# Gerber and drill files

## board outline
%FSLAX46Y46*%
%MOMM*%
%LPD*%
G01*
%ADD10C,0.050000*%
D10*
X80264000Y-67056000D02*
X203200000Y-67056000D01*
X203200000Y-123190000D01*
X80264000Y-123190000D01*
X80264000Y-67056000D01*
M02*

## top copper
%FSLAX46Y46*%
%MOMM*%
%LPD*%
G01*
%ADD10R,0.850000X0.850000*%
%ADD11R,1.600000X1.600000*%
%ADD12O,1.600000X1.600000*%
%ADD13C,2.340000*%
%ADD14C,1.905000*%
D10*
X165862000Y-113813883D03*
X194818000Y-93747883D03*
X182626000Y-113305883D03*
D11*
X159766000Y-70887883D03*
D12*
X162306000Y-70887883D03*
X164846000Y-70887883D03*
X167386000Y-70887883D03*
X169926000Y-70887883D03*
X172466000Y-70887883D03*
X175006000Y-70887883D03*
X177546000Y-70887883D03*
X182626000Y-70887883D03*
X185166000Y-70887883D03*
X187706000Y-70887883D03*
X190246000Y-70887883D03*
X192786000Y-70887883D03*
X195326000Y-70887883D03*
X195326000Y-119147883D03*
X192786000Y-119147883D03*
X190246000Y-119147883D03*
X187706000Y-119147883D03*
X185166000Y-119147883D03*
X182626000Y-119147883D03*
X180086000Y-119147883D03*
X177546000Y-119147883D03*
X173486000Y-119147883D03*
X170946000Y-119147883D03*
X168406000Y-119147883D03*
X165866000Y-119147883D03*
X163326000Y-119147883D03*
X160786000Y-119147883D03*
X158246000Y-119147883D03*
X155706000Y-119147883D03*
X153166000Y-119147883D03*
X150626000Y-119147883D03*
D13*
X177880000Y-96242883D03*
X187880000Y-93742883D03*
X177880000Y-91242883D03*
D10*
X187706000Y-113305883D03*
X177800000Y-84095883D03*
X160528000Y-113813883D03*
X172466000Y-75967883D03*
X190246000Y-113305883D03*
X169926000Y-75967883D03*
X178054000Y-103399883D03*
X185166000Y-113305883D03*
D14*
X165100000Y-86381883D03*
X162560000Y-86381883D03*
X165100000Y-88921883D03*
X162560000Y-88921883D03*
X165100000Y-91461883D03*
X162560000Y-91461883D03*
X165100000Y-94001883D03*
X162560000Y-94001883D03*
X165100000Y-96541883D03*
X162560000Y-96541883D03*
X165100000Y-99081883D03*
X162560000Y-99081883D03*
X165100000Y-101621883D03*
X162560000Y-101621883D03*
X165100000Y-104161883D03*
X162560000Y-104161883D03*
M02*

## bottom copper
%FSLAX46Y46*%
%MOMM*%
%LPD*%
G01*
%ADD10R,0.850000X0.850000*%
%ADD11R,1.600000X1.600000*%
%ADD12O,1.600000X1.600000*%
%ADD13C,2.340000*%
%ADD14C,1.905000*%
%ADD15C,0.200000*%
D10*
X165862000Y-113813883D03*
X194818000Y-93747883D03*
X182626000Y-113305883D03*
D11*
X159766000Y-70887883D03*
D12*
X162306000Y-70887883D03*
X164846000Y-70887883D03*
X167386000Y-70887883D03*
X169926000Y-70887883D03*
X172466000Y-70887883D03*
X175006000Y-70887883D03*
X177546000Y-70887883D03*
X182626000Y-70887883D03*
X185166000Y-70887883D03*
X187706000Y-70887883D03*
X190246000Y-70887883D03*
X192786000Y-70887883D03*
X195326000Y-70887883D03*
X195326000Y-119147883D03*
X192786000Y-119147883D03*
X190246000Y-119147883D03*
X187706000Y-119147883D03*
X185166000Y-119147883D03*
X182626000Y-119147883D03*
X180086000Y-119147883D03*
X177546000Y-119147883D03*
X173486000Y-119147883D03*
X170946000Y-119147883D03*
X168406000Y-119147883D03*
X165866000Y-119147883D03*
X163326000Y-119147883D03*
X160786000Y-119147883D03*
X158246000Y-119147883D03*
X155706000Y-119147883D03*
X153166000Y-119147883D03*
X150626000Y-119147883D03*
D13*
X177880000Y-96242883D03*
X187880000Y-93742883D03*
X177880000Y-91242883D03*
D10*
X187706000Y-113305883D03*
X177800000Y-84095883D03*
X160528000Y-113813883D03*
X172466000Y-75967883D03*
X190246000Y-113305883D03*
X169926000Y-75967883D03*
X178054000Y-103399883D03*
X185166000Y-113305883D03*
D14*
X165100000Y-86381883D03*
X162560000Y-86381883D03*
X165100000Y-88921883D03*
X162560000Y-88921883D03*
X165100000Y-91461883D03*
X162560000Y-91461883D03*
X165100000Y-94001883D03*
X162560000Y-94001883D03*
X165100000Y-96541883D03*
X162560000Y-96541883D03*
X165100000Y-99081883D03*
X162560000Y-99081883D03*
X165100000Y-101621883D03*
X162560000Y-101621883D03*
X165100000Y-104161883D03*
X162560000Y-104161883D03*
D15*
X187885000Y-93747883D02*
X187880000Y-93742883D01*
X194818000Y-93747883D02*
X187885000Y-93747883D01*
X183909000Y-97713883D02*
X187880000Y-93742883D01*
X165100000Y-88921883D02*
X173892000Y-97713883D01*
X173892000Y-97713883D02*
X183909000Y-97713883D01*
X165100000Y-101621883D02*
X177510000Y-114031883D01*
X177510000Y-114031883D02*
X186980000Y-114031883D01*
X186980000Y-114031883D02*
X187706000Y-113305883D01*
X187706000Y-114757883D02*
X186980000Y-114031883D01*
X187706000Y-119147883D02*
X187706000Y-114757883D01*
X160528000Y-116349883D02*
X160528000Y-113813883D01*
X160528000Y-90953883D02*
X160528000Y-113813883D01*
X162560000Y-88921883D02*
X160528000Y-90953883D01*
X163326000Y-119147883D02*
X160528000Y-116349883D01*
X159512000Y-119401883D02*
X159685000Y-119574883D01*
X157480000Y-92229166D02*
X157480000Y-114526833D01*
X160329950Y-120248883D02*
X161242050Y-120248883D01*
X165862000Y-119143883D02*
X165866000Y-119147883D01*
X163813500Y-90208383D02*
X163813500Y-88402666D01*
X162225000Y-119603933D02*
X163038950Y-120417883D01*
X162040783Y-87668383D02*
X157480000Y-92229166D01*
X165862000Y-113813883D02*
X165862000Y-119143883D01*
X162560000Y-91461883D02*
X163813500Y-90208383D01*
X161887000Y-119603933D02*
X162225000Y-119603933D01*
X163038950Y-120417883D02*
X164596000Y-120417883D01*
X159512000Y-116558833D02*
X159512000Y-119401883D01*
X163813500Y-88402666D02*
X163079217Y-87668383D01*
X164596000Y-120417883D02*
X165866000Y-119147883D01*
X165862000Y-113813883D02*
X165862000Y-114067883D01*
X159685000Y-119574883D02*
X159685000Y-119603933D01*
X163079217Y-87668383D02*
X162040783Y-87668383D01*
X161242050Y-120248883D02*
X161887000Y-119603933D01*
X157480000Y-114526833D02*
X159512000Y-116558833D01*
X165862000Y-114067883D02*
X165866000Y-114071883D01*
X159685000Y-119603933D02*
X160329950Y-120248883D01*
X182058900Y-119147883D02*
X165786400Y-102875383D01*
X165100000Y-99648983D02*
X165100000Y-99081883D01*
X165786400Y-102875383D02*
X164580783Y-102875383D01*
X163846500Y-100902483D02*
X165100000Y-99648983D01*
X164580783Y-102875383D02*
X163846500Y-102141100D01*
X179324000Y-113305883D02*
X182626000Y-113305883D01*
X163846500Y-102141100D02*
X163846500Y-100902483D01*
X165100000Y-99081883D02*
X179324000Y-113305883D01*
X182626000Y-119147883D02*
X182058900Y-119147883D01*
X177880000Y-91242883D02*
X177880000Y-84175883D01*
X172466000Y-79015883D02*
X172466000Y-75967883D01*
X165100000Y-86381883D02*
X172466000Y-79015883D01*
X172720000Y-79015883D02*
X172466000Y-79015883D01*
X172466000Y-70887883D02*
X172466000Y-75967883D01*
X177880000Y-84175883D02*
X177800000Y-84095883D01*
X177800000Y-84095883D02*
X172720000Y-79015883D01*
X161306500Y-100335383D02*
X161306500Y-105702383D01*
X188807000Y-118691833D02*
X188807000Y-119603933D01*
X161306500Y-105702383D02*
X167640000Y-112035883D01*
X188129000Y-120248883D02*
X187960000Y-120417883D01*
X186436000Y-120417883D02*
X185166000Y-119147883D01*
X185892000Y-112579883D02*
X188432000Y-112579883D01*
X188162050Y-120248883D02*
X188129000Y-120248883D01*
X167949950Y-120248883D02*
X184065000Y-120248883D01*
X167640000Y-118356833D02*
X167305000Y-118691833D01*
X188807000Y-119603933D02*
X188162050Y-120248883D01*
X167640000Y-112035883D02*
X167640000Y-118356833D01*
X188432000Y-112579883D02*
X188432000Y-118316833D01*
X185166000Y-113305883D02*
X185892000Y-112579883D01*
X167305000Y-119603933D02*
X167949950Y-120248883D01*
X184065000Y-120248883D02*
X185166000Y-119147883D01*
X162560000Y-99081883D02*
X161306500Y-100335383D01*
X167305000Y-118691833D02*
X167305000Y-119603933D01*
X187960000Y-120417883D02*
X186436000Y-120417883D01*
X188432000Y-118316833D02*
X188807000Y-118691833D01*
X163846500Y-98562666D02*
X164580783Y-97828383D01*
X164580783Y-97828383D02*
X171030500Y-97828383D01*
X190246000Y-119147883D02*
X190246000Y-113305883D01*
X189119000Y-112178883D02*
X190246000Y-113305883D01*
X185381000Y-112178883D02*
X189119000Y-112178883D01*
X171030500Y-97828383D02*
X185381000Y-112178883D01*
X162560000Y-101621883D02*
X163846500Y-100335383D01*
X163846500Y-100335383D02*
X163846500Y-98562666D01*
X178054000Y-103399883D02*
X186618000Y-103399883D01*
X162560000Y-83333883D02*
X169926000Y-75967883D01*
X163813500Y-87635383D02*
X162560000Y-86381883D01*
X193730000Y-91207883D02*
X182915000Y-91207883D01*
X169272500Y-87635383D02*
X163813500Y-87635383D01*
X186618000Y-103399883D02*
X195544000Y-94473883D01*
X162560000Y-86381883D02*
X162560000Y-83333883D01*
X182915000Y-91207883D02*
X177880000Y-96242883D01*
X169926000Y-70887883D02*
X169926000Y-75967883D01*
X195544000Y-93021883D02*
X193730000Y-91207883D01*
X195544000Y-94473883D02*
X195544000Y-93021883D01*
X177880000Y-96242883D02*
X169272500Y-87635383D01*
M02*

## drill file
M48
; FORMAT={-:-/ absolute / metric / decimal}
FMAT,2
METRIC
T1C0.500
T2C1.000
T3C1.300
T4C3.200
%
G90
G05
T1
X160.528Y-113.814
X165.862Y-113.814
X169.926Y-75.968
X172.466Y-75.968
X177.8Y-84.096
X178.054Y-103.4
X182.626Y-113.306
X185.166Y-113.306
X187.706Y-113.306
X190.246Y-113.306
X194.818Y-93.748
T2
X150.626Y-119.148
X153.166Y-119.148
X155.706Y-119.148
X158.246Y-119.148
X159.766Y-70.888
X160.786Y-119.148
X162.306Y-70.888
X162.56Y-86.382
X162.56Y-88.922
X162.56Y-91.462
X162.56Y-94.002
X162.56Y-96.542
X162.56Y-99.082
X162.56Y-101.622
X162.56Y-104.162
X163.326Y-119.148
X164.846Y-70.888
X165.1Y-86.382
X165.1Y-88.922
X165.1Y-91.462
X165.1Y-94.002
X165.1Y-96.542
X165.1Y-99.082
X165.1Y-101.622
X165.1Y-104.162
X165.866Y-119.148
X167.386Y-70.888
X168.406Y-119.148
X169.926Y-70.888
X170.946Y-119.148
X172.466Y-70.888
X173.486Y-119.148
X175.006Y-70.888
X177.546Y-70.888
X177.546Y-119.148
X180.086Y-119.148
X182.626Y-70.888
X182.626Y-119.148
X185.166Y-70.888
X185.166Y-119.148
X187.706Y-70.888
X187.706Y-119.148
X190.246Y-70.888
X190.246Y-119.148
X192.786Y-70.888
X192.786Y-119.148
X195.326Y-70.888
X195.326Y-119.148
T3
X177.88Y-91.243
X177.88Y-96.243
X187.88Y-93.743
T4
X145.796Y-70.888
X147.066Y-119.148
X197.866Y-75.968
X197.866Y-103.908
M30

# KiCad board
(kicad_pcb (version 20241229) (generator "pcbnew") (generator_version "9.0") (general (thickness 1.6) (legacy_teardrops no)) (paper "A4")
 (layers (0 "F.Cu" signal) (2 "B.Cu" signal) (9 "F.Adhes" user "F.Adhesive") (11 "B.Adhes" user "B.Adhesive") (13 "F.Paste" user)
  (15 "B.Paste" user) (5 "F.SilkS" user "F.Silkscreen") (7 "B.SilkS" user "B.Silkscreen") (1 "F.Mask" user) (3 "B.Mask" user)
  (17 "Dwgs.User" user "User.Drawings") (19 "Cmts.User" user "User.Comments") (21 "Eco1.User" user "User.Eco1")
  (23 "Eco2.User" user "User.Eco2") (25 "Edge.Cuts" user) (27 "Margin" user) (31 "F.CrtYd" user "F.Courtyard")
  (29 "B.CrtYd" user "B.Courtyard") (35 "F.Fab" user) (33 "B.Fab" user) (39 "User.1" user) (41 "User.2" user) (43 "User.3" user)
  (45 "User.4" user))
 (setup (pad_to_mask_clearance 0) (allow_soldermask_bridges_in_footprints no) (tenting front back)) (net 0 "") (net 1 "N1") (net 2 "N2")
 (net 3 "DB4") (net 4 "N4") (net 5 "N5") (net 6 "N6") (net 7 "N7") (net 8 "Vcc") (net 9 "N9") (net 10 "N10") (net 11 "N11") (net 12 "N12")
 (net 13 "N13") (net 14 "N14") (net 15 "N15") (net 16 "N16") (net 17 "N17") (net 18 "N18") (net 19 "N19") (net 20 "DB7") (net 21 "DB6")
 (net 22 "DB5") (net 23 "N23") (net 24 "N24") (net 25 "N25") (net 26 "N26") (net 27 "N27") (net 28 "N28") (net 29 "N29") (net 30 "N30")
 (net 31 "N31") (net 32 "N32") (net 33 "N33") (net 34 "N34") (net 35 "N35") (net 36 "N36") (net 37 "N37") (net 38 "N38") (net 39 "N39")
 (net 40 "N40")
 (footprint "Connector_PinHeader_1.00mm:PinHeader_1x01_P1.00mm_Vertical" (layer "F.Cu") (at 165.862 113.813883)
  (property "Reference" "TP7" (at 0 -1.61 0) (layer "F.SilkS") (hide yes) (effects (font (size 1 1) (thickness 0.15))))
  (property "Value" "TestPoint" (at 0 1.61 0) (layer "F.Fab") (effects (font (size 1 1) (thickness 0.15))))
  (pad "1" thru_hole rect (at 0 0) (size 0.85 0.85) (drill 0.5) (layers "*.Cu" "*.Mask") (remove_unused_layers no) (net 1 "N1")))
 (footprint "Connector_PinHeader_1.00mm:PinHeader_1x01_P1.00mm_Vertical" (layer "F.Cu") (at 194.818 93.747883)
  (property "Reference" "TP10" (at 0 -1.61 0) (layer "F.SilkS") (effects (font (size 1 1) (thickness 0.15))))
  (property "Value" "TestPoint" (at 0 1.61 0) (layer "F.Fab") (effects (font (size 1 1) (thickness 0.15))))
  (pad "1" thru_hole rect (at 0 0) (size 0.85 0.85) (drill 0.5) (layers "*.Cu" "*.Mask") (remove_unused_layers no) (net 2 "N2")))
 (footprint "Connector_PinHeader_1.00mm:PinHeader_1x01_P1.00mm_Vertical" (layer "F.Cu") (at 182.626 113.305883)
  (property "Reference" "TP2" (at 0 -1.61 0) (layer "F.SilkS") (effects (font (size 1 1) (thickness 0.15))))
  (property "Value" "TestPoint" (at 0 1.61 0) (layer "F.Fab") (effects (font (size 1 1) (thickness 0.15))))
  (pad "1" thru_hole rect (at 0 0) (size 0.85 0.85) (drill 0.5) (layers "*.Cu" "*.Mask") (remove_unused_layers no) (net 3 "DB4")))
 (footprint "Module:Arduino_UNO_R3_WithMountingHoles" (layer "F.Cu") (at 159.766 70.887883)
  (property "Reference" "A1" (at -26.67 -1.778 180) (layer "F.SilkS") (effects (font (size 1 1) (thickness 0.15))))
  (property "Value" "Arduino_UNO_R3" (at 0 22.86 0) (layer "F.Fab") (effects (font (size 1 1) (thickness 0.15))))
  (pad "" np_thru_hole circle (at -13.97 0 90) (size 3.2 3.2) (drill 3.2) (layers "*.Cu" "*.Mask"))
  (pad "" np_thru_hole circle (at -12.7 48.26 90) (size 3.2 3.2) (drill 3.2) (layers "*.Cu" "*.Mask"))
  (pad "" np_thru_hole circle (at 38.1 5.08 90) (size 3.2 3.2) (drill 3.2) (layers "*.Cu" "*.Mask"))
  (pad "" np_thru_hole circle (at 38.1 33.02 90) (size 3.2 3.2) (drill 3.2) (layers "*.Cu" "*.Mask"))
  (pad "1" thru_hole rect (at 0 0 90) (size 1.6 1.6) (drill 1) (layers "*.Cu" "*.Mask") (remove_unused_layers no) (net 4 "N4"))
  (pad "2" thru_hole oval (at 2.54 0 90) (size 1.6 1.6) (drill 1) (layers "*.Cu" "*.Mask") (remove_unused_layers no) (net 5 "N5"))
  (pad "3" thru_hole oval (at 5.08 0 90) (size 1.6 1.6) (drill 1) (layers "*.Cu" "*.Mask") (remove_unused_layers no) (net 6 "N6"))
  (pad "4" thru_hole oval (at 7.62 0 90) (size 1.6 1.6) (drill 1) (layers "*.Cu" "*.Mask") (remove_unused_layers no) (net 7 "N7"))
  (pad "5" thru_hole oval (at 10.16 0 90) (size 1.6 1.6) (drill 1) (layers "*.Cu" "*.Mask") (remove_unused_layers no) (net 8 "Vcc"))
  (pad "6" thru_hole oval (at 12.7 0 90) (size 1.6 1.6) (drill 1) (layers "*.Cu" "*.Mask") (remove_unused_layers no) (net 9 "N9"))
  (pad "7" thru_hole oval (at 15.24 0 90) (size 1.6 1.6) (drill 1) (layers "*.Cu" "*.Mask") (remove_unused_layers no) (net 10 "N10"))
  (pad "8" thru_hole oval (at 17.78 0 90) (size 1.6 1.6) (drill 1) (layers "*.Cu" "*.Mask") (remove_unused_layers no) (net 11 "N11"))
  (pad "9" thru_hole oval (at 22.86 0 90) (size 1.6 1.6) (drill 1) (layers "*.Cu" "*.Mask") (remove_unused_layers no) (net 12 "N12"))
  (pad "10" thru_hole oval (at 25.4 0 90) (size 1.6 1.6) (drill 1) (layers "*.Cu" "*.Mask") (remove_unused_layers no) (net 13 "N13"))
  (pad "11" thru_hole oval (at 27.94 0 90) (size 1.6 1.6) (drill 1) (layers "*.Cu" "*.Mask") (remove_unused_layers no) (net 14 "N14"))
  (pad "12" thru_hole oval (at 30.48 0 90) (size 1.6 1.6) (drill 1) (layers "*.Cu" "*.Mask") (remove_unused_layers no) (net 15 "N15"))
  (pad "13" thru_hole oval (at 33.02 0 90) (size 1.6 1.6) (drill 1) (layers "*.Cu" "*.Mask") (remove_unused_layers no) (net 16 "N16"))
  (pad "14" thru_hole oval (at 35.56 0 90) (size 1.6 1.6) (drill 1) (layers "*.Cu" "*.Mask") (remove_unused_layers no) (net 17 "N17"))
  (pad "15" thru_hole oval (at 35.56 48.26 90) (size 1.6 1.6) (drill 1) (layers "*.Cu" "*.Mask") (remove_unused_layers no) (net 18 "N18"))
  (pad "16" thru_hole oval (at 33.02 48.26 90) (size 1.6 1.6) (drill 1) (layers "*.Cu" "*.Mask") (remove_unused_layers no) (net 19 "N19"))
  (pad "17" thru_hole oval (at 30.48 48.26 90) (size 1.6 1.6) (drill 1) (layers "*.Cu" "*.Mask") (remove_unused_layers no) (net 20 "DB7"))
  (pad "18" thru_hole oval (at 27.94 48.26 90) (size 1.6 1.6) (drill 1) (layers "*.Cu" "*.Mask") (remove_unused_layers no) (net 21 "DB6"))
  (pad "19" thru_hole oval (at 25.4 48.26 90) (size 1.6 1.6) (drill 1) (layers "*.Cu" "*.Mask") (remove_unused_layers no) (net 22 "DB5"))
  (pad "20" thru_hole oval (at 22.86 48.26 90) (size 1.6 1.6) (drill 1) (layers "*.Cu" "*.Mask") (remove_unused_layers no) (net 3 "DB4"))
  (pad "21" thru_hole oval (at 20.32 48.26 90) (size 1.6 1.6) (drill 1) (layers "*.Cu" "*.Mask") (remove_unused_layers no) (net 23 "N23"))
  (pad "22" thru_hole oval (at 17.78 48.26 90) (size 1.6 1.6) (drill 1) (layers "*.Cu" "*.Mask") (remove_unused_layers no) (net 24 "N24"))
  (pad "23" thru_hole oval (at 13.72 48.26 90) (size 1.6 1.6) (drill 1) (layers "*.Cu" "*.Mask") (remove_unused_layers no) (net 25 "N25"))
  (pad "24" thru_hole oval (at 11.18 48.26 90) (size 1.6 1.6) (drill 1) (layers "*.Cu" "*.Mask") (remove_unused_layers no) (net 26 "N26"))
  (pad "25" thru_hole oval (at 8.64 48.26 90) (size 1.6 1.6) (drill 1) (layers "*.Cu" "*.Mask") (remove_unused_layers no) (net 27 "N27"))
  (pad "26" thru_hole oval (at 6.1 48.26 90) (size 1.6 1.6) (drill 1) (layers "*.Cu" "*.Mask") (remove_unused_layers no) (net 1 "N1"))
  (pad "27" thru_hole oval (at 3.56 48.26 90) (size 1.6 1.6) (drill 1) (layers "*.Cu" "*.Mask") (remove_unused_layers no) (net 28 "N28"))
  (pad "28" thru_hole oval (at 1.02 48.26 90) (size 1.6 1.6) (drill 1) (layers "*.Cu" "*.Mask") (remove_unused_layers no) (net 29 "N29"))
  (pad "29" thru_hole oval (at -1.52 48.26 90) (size 1.6 1.6) (drill 1) (layers "*.Cu" "*.Mask") (remove_unused_layers no) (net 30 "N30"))
  (pad "30" thru_hole oval (at -4.06 48.26 90) (size 1.6 1.6) (drill 1) (layers "*.Cu" "*.Mask") (remove_unused_layers no) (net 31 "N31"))
  (pad "31" thru_hole oval (at -6.6 48.26 90) (size 1.6 1.6) (drill 1) (layers "*.Cu" "*.Mask") (remove_unused_layers no) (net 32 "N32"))
  (pad "32" thru_hole oval (at -9.14 48.26 90) (size 1.6 1.6) (drill 1) (layers "*.Cu" "*.Mask") (remove_unused_layers no) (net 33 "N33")))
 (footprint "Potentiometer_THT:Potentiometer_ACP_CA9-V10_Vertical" (layer "F.Cu") (at 177.88 96.242883)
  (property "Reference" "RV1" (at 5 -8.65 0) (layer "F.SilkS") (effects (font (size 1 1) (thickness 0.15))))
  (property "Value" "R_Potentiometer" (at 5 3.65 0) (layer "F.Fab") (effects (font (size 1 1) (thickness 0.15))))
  (pad "1" thru_hole circle (at 0 0) (size 2.34 2.34) (drill 1.3) (layers "*.Cu" "*.Mask") (remove_unused_layers no) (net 8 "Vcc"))
  (pad "2" thru_hole circle (at 10 -2.5) (size 2.34 2.34) (drill 1.3) (layers "*.Cu" "*.Mask") (remove_unused_layers no) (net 2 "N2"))
  (pad "3" thru_hole circle (at 0 -5) (size 2.34 2.34) (drill 1.3) (layers "*.Cu" "*.Mask") (remove_unused_layers no) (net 9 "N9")))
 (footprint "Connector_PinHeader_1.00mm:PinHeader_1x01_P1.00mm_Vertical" (layer "F.Cu") (at 187.706 113.305883)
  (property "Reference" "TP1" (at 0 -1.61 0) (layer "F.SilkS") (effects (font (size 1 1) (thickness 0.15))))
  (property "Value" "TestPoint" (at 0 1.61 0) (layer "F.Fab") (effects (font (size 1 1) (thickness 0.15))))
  (pad "1" thru_hole rect (at 0 0) (size 0.85 0.85) (drill 0.5) (layers "*.Cu" "*.Mask") (remove_unused_layers no) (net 21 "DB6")))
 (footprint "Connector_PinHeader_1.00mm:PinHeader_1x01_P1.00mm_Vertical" (layer "F.Cu") (at 177.8 84.095883)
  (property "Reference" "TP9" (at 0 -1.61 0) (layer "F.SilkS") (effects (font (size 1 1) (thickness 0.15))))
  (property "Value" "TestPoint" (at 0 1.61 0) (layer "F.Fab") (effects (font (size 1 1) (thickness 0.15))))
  (pad "1" thru_hole rect (at 0 0) (size 0.85 0.85) (drill 0.5) (layers "*.Cu" "*.Mask") (remove_unused_layers no) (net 9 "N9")))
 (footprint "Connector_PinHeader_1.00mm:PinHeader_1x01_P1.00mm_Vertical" (layer "F.Cu") (at 160.528 113.813883)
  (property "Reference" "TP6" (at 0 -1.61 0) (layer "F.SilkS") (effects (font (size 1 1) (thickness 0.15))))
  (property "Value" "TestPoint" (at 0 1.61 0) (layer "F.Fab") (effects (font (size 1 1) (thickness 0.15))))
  (pad "1" thru_hole rect (at 0 0) (size 0.85 0.85) (drill 0.5) (layers "*.Cu" "*.Mask") (remove_unused_layers no) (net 28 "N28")))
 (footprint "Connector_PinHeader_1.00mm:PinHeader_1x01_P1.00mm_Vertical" (layer "F.Cu") (at 172.466 75.967883)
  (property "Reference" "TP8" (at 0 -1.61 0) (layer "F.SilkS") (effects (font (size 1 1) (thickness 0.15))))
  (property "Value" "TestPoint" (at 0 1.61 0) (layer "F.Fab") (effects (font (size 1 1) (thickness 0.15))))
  (pad "1" thru_hole rect (at 0 0) (size 0.85 0.85) (drill 0.5) (layers "*.Cu" "*.Mask") (remove_unused_layers no) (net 9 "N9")))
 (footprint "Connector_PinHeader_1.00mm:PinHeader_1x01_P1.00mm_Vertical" (layer "F.Cu") (at 190.246 113.305883)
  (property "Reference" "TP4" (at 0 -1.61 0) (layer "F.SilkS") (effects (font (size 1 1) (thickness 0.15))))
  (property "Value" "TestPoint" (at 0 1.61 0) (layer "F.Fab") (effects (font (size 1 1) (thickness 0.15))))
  (pad "1" thru_hole rect (at 0 0) (size 0.85 0.85) (drill 0.5) (layers "*.Cu" "*.Mask") (remove_unused_layers no) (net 20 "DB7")))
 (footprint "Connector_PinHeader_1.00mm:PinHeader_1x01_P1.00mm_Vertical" (layer "F.Cu") (at 169.926 75.967883)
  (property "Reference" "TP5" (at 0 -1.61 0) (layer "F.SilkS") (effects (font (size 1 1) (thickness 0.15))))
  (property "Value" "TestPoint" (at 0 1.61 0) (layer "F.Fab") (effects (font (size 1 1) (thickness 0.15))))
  (pad "1" thru_hole rect (at 0 0) (size 0.85 0.85) (drill 0.5) (layers "*.Cu" "*.Mask") (remove_unused_layers no) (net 8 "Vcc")))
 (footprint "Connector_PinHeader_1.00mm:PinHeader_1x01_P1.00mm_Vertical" (layer "F.Cu") (at 178.054 103.399883)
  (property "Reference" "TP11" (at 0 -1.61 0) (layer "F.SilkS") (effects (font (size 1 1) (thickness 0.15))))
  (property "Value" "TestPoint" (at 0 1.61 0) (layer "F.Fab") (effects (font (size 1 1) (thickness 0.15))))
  (pad "1" thru_hole rect (at 0 0) (size 0.85 0.85) (drill 0.5) (layers "*.Cu" "*.Mask") (remove_unused_layers no) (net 8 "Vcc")))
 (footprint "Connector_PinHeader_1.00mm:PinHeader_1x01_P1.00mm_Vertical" (layer "F.Cu") (at 185.166 113.305883)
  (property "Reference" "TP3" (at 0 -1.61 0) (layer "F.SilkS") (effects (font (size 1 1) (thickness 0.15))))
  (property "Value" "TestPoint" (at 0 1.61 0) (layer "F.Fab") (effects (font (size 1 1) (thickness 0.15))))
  (pad "1" thru_hole rect (at 0 0) (size 0.85 0.85) (drill 0.5) (layers "*.Cu" "*.Mask") (remove_unused_layers no) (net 22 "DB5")))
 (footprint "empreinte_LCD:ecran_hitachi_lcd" (layer "F.Cu") (at 124.46 94.001883 180)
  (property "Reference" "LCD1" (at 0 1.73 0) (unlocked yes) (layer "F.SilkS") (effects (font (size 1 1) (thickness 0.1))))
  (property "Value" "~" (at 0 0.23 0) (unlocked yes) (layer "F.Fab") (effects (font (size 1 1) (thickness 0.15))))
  (pad "1" thru_hole circle (at -40.64 7.62 180) (size 1.905 1.905) (drill 1) (layers "*.Cu" "F.Mask" "F.Paste") (remove_unused_layers no)
   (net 9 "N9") (thermal_bridge_angle 90))
  (pad "2" thru_hole circle (at -38.1 7.62 180) (size 1.905 1.905) (drill 1) (layers "*.Cu" "F.Mask" "F.Paste") (remove_unused_layers no)
   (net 8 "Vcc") (thermal_bridge_angle 90))
  (pad "3" thru_hole circle (at -40.64 5.08 180) (size 1.905 1.905) (drill 1) (layers "*.Cu" "F.Mask" "F.Paste") (remove_unused_layers no)
   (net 2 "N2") (thermal_bridge_angle 90))
  (pad "4" thru_hole circle (at -38.1 5.08 180) (size 1.905 1.905) (drill 1) (layers "*.Cu" "F.Mask" "F.Paste") (remove_unused_layers no)
   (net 28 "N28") (thermal_bridge_angle 90))
  (pad "5" thru_hole circle (at -40.64 2.54 180) (size 1.905 1.905) (drill 1) (layers "*.Cu" "F.Mask" "F.Paste") (remove_unused_layers no)
   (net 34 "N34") (thermal_bridge_angle 90))
  (pad "6" thru_hole circle (at -38.1 2.54 180) (size 1.905 1.905) (drill 1) (layers "*.Cu" "F.Mask" "F.Paste") (remove_unused_layers no)
   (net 1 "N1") (thermal_bridge_angle 90))
  (pad "7" thru_hole circle (at -40.64 0 180) (size 1.905 1.905) (drill 1) (layers "*.Cu" "F.Mask" "F.Paste") (remove_unused_layers no)
   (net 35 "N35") (thermal_bridge_angle 90))
  (pad "8" thru_hole circle (at -38.1 0 180) (size 1.905 1.905) (drill 1) (layers "*.Cu" "F.Mask" "F.Paste") (remove_unused_layers no)
   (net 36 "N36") (thermal_bridge_angle 90))
  (pad "9" thru_hole circle (at -40.64 -2.54 180) (size 1.905 1.905) (drill 1) (layers "*.Cu" "F.Mask" "F.Paste") (remove_unused_layers no)
   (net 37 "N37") (thermal_bridge_angle 90))
  (pad "10" thru_hole circle (at -38.1 -2.54 180) (size 1.905 1.905) (drill 1) (layers "*.Cu" "F.Mask" "F.Paste") (remove_unused_layers no)
   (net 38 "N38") (thermal_bridge_angle 90))
  (pad "11" thru_hole circle (at -40.64 -5.08 180) (size 1.905 1.905) (drill 1) (layers "*.Cu" "F.Mask" "F.Paste") (remove_unused_layers no)
   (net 3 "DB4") (thermal_bridge_angle 90))
  (pad "12" thru_hole circle (at -38.1 -5.08 180) (size 1.905 1.905) (drill 1) (layers "*.Cu" "F.Mask" "F.Paste") (remove_unused_layers no)
   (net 22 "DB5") (thermal_bridge_angle 90))
  (pad "13" thru_hole circle (at -40.64 -7.62 180) (size 1.905 1.905) (drill 1) (layers "*.Cu" "F.Mask" "F.Paste") (remove_unused_layers no)
   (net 21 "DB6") (thermal_bridge_angle 90))
  (pad "14" thru_hole circle (at -38.1 -7.62 180) (size 1.905 1.905) (drill 1) (layers "*.Cu" "F.Mask" "F.Paste") (remove_unused_layers no)
   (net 20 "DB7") (thermal_bridge_angle 90))
  (pad "15" thru_hole circle (at -40.64 -10.16 180) (size 1.905 1.905) (drill 1) (layers "*.Cu" "F.Mask" "F.Paste")
   (remove_unused_layers no) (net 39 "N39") (thermal_bridge_angle 90))
  (pad "16" thru_hole circle (at -38.1 -10.16 180) (size 1.905 1.905) (drill 1) (layers "*.Cu" "F.Mask" "F.Paste") (remove_unused_layers no)
   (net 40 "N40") (thermal_bridge_angle 90)))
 (gr_rect (start 80.264 67.056) (end 203.2 123.19) (stroke (width 0.05) (type default)) (fill no) (layer "Edge.Cuts"))
 (segment (start 187.885 93.747883) (end 187.88 93.742883) (width 0.2) (layer "B.Cu") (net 2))
 (segment (start 194.818 93.747883) (end 187.885 93.747883) (width 0.2) (layer "B.Cu") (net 2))
 (segment (start 183.909 97.713883) (end 187.88 93.742883) (width 0.2) (layer "B.Cu") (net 2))
 (segment (start 165.1 88.921883) (end 173.892 97.713883) (width 0.2) (layer "B.Cu") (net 2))
 (segment (start 173.892 97.713883) (end 183.909 97.713883) (width 0.2) (layer "B.Cu") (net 2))
 (segment (start 165.1 101.621883) (end 177.51 114.031883) (width 0.2) (layer "B.Cu") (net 21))
 (segment (start 177.51 114.031883) (end 186.98 114.031883) (width 0.2) (layer "B.Cu") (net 21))
 (segment (start 186.98 114.031883) (end 187.706 113.305883) (width 0.2) (layer "B.Cu") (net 21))
 (segment (start 187.706 114.757883) (end 186.98 114.031883) (width 0.2) (layer "B.Cu") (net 21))
 (segment (start 187.706 119.147883) (end 187.706 114.757883) (width 0.2) (layer "B.Cu") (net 21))
 (segment (start 160.528 116.349883) (end 160.528 113.813883) (width 0.2) (layer "B.Cu") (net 28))
 (segment (start 160.528 90.953883) (end 160.528 113.813883) (width 0.2) (layer "B.Cu") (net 28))
 (segment (start 162.56 88.921883) (end 160.528 90.953883) (width 0.2) (layer "B.Cu") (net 28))
 (segment (start 163.326 119.147883) (end 160.528 116.349883) (width 0.2) (layer "B.Cu") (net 28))
 (segment (start 159.512 119.401883) (end 159.685 119.574883) (width 0.2) (layer "B.Cu") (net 1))
 (segment (start 157.48 92.229166) (end 157.48 114.526833) (width 0.2) (layer "B.Cu") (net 1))
 (segment (start 160.32995 120.248883) (end 161.24205 120.248883) (width 0.2) (layer "B.Cu") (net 1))
 (segment (start 165.862 119.143883) (end 165.866 119.147883) (width 0.2) (layer "B.Cu") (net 1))
 (segment (start 163.8135 90.208383) (end 163.8135 88.402666) (width 0.2) (layer "B.Cu") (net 1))
 (segment (start 162.225 119.603933) (end 163.03895 120.417883) (width 0.2) (layer "B.Cu") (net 1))
 (segment (start 162.040783 87.668383) (end 157.48 92.229166) (width 0.2) (layer "B.Cu") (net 1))
 (segment (start 165.862 113.813883) (end 165.862 119.143883) (width 0.2) (layer "B.Cu") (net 1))
 (segment (start 162.56 91.461883) (end 163.8135 90.208383) (width 0.2) (layer "B.Cu") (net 1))
 (segment (start 161.887 119.603933) (end 162.225 119.603933) (width 0.2) (layer "B.Cu") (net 1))
 (segment (start 163.03895 120.417883) (end 164.596 120.417883) (width 0.2) (layer "B.Cu") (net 1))
 (segment (start 159.512 116.558833) (end 159.512 119.401883) (width 0.2) (layer "B.Cu") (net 1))
 (segment (start 163.8135 88.402666) (end 163.079217 87.668383) (width 0.2) (layer "B.Cu") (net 1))
 (segment (start 164.596 120.417883) (end 165.866 119.147883) (width 0.2) (layer "B.Cu") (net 1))
 (segment (start 165.862 113.813883) (end 165.862 114.067883) (width 0.2) (layer "B.Cu") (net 1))
 (segment (start 159.685 119.574883) (end 159.685 119.603933) (width 0.2) (layer "B.Cu") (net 1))
 (segment (start 163.079217 87.668383) (end 162.040783 87.668383) (width 0.2) (layer "B.Cu") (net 1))
 (segment (start 161.24205 120.248883) (end 161.887 119.603933) (width 0.2) (layer "B.Cu") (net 1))
 (segment (start 157.48 114.526833) (end 159.512 116.558833) (width 0.2) (layer "B.Cu") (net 1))
 (segment (start 165.862 114.067883) (end 165.866 114.071883) (width 0.2) (layer "B.Cu") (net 1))
 (segment (start 159.685 119.603933) (end 160.32995 120.248883) (width 0.2) (layer "B.Cu") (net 1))
 (segment (start 182.0589 119.147883) (end 165.7864 102.875383) (width 0.2) (layer "B.Cu") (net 3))
 (segment (start 165.1 99.648983) (end 165.1 99.081883) (width 0.2) (layer "B.Cu") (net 3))
 (segment (start 165.7864 102.875383) (end 164.580783 102.875383) (width 0.2) (layer "B.Cu") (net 3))
 (segment (start 163.8465 100.902483) (end 165.1 99.648983) (width 0.2) (layer "B.Cu") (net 3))
 (segment (start 164.580783 102.875383) (end 163.8465 102.1411) (width 0.2) (layer "B.Cu") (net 3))
 (segment (start 179.324 113.305883) (end 182.626 113.305883) (width 0.2) (layer "B.Cu") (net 3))
 (segment (start 163.8465 102.1411) (end 163.8465 100.902483) (width 0.2) (layer "B.Cu") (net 3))
 (segment (start 165.1 99.081883) (end 179.324 113.305883) (width 0.2) (layer "B.Cu") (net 3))
 (segment (start 182.626 119.147883) (end 182.0589 119.147883) (width 0.2) (layer "B.Cu") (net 3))
 (segment (start 177.88 91.242883) (end 177.88 84.175883) (width 0.2) (layer "B.Cu") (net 9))
 (segment (start 172.466 79.015883) (end 172.466 75.967883) (width 0.2) (layer "B.Cu") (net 9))
 (segment (start 165.1 86.381883) (end 172.466 79.015883) (width 0.2) (layer "B.Cu") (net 9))
 (segment (start 172.72 79.015883) (end 172.466 79.015883) (width 0.2) (layer "B.Cu") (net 9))
 (segment (start 172.466 70.887883) (end 172.466 75.967883) (width 0.2) (layer "B.Cu") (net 9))
 (segment (start 177.88 84.175883) (end 177.8 84.095883) (width 0.2) (layer "B.Cu") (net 9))
 (segment (start 177.8 84.095883) (end 172.72 79.015883) (width 0.2) (layer "B.Cu") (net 9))
 (segment (start 161.3065 100.335383) (end 161.3065 105.702383) (width 0.2) (layer "B.Cu") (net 22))
 (segment (start 188.807 118.691833) (end 188.807 119.603933) (width 0.2) (layer "B.Cu") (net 22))
 (segment (start 161.3065 105.702383) (end 167.64 112.035883) (width 0.2) (layer "B.Cu") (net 22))
 (segment (start 188.129 120.248883) (end 187.96 120.417883) (width 0.2) (layer "B.Cu") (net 22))
 (segment (start 186.436 120.417883) (end 185.166 119.147883) (width 0.2) (layer "B.Cu") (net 22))
 (segment (start 185.892 112.579883) (end 188.432 112.579883) (width 0.2) (layer "B.Cu") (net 22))
 (segment (start 188.16205 120.248883) (end 188.129 120.248883) (width 0.2) (layer "B.Cu") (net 22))
 (segment (start 167.94995 120.248883) (end 184.065 120.248883) (width 0.2) (layer "B.Cu") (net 22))
 (segment (start 167.64 118.356833) (end 167.305 118.691833) (width 0.2) (layer "B.Cu") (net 22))
 (segment (start 188.807 119.603933) (end 188.16205 120.248883) (width 0.2) (layer "B.Cu") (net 22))
 (segment (start 167.64 112.035883) (end 167.64 118.356833) (width 0.2) (layer "B.Cu") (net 22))
 (segment (start 188.432 112.579883) (end 188.432 118.316833) (width 0.2) (layer "B.Cu") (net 22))
 (segment (start 185.166 113.305883) (end 185.892 112.579883) (width 0.2) (layer "B.Cu") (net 22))
 (segment (start 167.305 119.603933) (end 167.94995 120.248883) (width 0.2) (layer "B.Cu") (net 22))
 (segment (start 184.065 120.248883) (end 185.166 119.147883) (width 0.2) (layer "B.Cu") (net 22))
 (segment (start 162.56 99.081883) (end 161.3065 100.335383) (width 0.2) (layer "B.Cu") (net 22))
 (segment (start 167.305 118.691833) (end 167.305 119.603933) (width 0.2) (layer "B.Cu") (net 22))
 (segment (start 187.96 120.417883) (end 186.436 120.417883) (width 0.2) (layer "B.Cu") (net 22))
 (segment (start 188.432 118.316833) (end 188.807 118.691833) (width 0.2) (layer "B.Cu") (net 22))
 (segment (start 163.8465 98.562666) (end 164.580783 97.828383) (width 0.2) (layer "B.Cu") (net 20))
 (segment (start 164.580783 97.828383) (end 171.0305 97.828383) (width 0.2) (layer "B.Cu") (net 20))
 (segment (start 190.246 119.147883) (end 190.246 113.305883) (width 0.2) (layer "B.Cu") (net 20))
 (segment (start 189.119 112.178883) (end 190.246 113.305883) (width 0.2) (layer "B.Cu") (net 20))
 (segment (start 185.381 112.178883) (end 189.119 112.178883) (width 0.2) (layer "B.Cu") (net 20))
 (segment (start 171.0305 97.828383) (end 185.381 112.178883) (width 0.2) (layer "B.Cu") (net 20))
 (segment (start 162.56 101.621883) (end 163.8465 100.335383) (width 0.2) (layer "B.Cu") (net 20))
 (segment (start 163.8465 100.335383) (end 163.8465 98.562666) (width 0.2) (layer "B.Cu") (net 20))
 (segment (start 178.054 103.399883) (end 186.618 103.399883) (width 0.2) (layer "B.Cu") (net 8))
 (segment (start 162.56 83.333883) (end 169.926 75.967883) (width 0.2) (layer "B.Cu") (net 8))
 (segment (start 163.8135 87.635383) (end 162.56 86.381883) (width 0.2) (layer "B.Cu") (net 8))
 (segment (start 193.73 91.207883) (end 182.915 91.207883) (width 0.2) (layer "B.Cu") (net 8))
 (segment (start 169.2725 87.635383) (end 163.8135 87.635383) (width 0.2) (layer "B.Cu") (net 8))
 (segment (start 186.618 103.399883) (end 195.544 94.473883) (width 0.2) (layer "B.Cu") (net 8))
 (segment (start 162.56 86.381883) (end 162.56 83.333883) (width 0.2) (layer "B.Cu") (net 8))
 (segment (start 182.915 91.207883) (end 177.88 96.242883) (width 0.2) (layer "B.Cu") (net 8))
 (segment (start 169.926 70.887883) (end 169.926 75.967883) (width 0.2) (layer "B.Cu") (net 8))
 (segment (start 195.544 93.021883) (end 193.73 91.207883) (width 0.2) (layer "B.Cu") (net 8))
 (segment (start 195.544 94.473883) (end 195.544 93.021883) (width 0.2) (layer "B.Cu") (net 8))
 (segment (start 177.88 96.242883) (end 169.2725 87.635383) (width 0.2) (layer "B.Cu") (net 8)))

